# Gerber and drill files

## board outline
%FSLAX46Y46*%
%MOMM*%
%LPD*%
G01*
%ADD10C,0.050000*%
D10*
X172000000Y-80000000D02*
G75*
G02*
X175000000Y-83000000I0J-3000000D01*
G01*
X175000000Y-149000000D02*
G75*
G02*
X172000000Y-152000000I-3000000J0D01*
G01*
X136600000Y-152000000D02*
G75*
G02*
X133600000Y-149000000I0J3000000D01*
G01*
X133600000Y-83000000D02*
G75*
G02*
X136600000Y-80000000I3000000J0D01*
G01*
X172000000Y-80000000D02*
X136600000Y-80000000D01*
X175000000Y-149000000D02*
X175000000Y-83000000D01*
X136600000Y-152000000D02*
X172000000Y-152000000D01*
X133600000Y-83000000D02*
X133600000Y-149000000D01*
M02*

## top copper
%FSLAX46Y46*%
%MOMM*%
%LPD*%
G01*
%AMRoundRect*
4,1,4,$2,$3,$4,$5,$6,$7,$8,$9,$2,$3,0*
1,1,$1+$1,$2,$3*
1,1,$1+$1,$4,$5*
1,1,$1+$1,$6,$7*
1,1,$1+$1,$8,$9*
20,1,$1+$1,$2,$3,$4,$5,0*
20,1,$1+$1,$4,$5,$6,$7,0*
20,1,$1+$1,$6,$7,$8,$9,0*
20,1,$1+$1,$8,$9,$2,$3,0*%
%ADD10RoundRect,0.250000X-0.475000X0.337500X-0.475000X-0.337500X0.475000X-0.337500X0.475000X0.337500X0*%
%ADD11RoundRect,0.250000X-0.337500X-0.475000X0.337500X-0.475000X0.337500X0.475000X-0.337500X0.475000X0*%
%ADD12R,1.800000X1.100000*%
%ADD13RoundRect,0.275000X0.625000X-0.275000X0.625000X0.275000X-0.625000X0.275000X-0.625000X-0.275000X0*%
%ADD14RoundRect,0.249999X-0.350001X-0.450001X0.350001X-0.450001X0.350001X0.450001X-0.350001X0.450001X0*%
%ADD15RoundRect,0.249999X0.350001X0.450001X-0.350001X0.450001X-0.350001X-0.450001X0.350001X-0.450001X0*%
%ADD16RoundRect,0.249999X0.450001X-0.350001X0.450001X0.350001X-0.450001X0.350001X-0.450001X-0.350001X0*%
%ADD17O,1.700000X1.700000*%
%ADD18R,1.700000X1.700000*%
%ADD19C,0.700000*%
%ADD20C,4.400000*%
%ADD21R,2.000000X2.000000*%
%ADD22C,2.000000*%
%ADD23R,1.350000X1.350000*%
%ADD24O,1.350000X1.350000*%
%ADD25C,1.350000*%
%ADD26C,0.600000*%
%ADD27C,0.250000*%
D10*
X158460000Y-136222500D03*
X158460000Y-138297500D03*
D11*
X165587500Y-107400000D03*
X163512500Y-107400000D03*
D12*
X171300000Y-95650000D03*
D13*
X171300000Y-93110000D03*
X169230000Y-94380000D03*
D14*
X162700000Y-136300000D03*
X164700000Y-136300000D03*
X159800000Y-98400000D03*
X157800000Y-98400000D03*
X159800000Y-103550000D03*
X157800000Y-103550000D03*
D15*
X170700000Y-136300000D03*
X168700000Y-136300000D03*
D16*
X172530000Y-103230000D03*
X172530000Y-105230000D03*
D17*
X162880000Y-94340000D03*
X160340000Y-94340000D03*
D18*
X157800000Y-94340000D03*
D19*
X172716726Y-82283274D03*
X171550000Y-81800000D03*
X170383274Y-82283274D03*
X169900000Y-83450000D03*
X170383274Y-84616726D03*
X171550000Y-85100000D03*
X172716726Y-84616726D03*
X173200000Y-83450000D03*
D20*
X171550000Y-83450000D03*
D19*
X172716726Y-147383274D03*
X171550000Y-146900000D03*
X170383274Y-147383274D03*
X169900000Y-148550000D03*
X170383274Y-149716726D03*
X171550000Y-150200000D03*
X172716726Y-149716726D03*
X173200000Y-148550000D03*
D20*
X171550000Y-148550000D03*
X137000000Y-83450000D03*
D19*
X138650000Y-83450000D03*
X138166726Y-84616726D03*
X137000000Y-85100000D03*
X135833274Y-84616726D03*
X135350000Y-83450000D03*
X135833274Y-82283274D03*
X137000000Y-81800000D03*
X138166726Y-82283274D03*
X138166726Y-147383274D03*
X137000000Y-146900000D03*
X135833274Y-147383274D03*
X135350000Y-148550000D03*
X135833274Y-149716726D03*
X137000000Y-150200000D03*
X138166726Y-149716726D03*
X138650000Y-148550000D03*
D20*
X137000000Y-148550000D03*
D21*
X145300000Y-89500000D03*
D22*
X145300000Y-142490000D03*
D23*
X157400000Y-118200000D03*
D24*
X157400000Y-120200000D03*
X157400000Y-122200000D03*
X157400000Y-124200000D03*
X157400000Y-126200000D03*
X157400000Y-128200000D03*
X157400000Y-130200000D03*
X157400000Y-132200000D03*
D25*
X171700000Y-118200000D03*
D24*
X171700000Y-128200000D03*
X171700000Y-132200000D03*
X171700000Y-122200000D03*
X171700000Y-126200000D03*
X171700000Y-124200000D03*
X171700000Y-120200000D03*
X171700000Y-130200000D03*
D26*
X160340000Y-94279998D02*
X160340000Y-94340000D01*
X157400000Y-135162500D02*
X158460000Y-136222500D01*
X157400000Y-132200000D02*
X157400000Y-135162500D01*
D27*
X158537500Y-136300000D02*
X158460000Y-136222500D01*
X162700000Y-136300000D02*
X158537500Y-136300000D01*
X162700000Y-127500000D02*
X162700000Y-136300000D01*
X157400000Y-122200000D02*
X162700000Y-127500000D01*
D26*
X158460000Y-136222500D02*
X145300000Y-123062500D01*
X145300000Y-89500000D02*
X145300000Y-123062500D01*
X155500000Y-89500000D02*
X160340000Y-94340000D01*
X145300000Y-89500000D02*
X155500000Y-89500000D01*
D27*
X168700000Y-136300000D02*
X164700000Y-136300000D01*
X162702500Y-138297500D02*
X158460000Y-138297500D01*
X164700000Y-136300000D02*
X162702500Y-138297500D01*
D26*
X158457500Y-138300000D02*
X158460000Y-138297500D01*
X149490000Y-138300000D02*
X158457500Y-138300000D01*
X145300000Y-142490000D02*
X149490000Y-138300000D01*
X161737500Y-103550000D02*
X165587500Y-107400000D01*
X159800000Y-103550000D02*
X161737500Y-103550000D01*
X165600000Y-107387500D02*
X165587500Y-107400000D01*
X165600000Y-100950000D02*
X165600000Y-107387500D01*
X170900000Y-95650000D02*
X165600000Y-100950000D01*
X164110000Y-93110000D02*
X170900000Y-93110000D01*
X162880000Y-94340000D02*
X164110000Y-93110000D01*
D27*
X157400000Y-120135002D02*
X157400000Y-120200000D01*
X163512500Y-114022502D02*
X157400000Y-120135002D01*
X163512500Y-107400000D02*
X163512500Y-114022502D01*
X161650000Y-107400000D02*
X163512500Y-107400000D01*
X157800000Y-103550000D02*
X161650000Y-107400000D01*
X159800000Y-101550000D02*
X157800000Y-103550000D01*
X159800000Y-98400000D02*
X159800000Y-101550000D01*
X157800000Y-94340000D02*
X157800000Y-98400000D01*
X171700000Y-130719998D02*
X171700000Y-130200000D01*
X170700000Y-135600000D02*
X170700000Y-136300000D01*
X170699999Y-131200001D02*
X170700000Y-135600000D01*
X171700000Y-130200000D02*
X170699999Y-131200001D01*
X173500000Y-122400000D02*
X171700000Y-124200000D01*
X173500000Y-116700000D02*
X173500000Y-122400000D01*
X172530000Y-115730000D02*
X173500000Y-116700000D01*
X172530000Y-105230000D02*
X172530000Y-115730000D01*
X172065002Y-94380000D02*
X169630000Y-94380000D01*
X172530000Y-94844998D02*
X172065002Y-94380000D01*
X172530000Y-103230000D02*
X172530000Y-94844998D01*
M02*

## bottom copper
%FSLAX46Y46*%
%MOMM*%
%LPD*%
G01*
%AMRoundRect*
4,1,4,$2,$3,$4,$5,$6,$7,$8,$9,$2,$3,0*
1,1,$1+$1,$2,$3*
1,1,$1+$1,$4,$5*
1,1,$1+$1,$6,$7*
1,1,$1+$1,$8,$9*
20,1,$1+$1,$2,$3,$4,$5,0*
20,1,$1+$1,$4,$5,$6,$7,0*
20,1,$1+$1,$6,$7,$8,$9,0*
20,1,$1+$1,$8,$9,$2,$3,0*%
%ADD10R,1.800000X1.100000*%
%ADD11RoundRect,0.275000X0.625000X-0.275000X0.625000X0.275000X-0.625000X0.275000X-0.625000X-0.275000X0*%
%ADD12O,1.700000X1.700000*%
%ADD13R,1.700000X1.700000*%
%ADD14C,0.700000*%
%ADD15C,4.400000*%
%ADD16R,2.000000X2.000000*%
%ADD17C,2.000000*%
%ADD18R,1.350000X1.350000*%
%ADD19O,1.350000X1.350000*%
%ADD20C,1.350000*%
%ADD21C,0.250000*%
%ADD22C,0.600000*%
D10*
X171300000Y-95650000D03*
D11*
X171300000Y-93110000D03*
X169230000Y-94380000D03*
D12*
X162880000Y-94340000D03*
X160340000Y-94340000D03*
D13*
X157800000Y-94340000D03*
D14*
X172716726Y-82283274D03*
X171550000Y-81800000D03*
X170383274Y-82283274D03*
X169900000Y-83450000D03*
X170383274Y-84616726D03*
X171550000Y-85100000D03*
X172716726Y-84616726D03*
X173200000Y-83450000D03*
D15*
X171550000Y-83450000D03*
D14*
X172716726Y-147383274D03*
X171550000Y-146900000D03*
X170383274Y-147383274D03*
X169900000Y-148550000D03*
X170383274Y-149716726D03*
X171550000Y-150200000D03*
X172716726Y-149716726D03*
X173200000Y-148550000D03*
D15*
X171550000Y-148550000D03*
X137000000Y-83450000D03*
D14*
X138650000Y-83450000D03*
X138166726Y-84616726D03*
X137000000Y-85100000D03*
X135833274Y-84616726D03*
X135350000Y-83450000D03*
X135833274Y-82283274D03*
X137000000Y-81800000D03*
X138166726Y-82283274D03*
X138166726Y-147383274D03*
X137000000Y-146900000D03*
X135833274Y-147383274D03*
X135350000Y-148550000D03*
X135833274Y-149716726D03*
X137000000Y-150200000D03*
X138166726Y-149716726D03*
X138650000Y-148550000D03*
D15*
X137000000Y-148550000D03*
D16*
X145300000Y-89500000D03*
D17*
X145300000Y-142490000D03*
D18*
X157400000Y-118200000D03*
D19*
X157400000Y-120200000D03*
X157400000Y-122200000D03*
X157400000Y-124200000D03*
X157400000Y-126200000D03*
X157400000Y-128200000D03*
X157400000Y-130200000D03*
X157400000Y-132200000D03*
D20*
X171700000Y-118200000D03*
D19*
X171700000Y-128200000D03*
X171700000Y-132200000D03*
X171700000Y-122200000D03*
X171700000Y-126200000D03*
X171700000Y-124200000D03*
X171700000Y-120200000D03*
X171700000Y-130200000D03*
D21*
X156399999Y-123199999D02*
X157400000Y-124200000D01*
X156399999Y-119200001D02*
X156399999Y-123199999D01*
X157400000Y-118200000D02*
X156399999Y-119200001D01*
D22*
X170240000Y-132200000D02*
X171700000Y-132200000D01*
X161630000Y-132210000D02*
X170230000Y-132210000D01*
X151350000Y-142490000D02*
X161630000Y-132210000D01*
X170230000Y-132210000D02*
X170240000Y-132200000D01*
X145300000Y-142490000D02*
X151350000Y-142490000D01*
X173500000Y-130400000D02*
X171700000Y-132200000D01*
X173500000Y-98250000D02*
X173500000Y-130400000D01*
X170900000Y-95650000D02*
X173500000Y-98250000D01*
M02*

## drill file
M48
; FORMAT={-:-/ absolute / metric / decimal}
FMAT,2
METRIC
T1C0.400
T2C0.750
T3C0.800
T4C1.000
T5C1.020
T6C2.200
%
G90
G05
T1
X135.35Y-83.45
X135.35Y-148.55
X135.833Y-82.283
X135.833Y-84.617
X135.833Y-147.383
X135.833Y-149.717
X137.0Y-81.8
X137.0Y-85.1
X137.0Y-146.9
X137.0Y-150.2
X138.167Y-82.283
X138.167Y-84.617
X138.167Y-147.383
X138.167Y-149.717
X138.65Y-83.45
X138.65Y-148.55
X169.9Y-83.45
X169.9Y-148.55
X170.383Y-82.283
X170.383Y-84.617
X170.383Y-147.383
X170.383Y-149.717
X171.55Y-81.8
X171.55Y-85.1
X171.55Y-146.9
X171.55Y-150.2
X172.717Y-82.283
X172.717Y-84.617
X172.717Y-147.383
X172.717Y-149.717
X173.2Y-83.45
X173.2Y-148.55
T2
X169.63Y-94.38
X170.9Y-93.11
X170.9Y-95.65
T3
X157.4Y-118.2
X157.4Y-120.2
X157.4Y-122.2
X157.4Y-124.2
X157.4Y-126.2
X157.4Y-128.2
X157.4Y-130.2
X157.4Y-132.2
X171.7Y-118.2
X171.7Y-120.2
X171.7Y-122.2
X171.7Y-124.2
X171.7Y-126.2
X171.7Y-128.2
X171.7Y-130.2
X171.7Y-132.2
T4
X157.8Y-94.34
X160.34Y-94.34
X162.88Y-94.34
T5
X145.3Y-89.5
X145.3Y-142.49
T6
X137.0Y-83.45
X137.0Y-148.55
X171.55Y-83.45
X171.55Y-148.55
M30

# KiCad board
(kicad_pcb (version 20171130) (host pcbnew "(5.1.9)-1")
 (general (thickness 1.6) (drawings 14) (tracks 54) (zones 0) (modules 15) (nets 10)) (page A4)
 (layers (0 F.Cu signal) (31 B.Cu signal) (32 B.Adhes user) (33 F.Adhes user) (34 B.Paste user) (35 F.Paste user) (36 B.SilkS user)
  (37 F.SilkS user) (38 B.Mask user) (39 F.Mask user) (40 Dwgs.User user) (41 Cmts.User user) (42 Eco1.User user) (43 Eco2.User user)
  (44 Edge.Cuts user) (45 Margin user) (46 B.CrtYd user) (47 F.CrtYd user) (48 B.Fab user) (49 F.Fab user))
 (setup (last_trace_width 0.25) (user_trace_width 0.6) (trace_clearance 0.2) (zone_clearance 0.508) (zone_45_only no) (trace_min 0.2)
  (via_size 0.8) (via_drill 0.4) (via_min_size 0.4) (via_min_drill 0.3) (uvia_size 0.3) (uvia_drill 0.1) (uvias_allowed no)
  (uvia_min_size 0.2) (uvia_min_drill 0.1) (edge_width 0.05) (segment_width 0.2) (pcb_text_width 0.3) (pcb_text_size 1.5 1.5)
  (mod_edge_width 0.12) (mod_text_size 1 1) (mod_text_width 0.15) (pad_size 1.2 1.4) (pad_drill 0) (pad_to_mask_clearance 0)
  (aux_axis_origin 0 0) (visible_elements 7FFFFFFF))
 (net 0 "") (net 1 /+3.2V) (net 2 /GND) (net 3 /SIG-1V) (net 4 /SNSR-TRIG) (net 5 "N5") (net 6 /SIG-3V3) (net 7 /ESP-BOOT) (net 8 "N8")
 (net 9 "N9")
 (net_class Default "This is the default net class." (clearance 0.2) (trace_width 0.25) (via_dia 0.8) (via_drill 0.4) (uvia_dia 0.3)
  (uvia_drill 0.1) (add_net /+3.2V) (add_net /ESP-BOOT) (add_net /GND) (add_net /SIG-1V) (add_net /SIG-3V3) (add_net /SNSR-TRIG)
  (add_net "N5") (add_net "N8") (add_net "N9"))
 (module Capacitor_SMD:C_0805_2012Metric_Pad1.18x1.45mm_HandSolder (layer F.Cu) (at 158.46 137.26 270)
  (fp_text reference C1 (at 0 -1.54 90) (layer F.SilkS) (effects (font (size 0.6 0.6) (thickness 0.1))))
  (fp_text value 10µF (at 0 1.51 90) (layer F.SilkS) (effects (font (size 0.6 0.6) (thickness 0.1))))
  (pad 1 smd roundrect (at -1.0375 0 270) (size 1.175 1.45) (layers F.Cu F.Paste F.Mask) (roundrect_rratio 0.2127659574468085)
   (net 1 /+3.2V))
  (pad 2 smd roundrect (at 1.0375 0 270) (size 1.175 1.45) (layers F.Cu F.Paste F.Mask) (roundrect_rratio 0.2127659574468085) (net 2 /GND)))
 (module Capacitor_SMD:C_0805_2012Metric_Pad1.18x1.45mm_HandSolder (layer F.Cu) (at 164.55 107.4)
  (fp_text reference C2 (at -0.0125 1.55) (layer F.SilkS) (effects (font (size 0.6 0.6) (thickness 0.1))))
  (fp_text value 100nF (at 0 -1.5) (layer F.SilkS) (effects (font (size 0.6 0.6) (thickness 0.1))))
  (pad 2 smd roundrect (at 1.0375 0) (size 1.175 1.45) (layers F.Cu F.Paste F.Mask) (roundrect_rratio 0.2127659574468085) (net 2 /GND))
  (pad 1 smd roundrect (at -1.0375 0) (size 1.175 1.45) (layers F.Cu F.Paste F.Mask) (roundrect_rratio 0.2127659574468085) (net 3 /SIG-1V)))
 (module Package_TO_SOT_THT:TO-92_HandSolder (layer F.Cu) (at 170.9 95.65 90)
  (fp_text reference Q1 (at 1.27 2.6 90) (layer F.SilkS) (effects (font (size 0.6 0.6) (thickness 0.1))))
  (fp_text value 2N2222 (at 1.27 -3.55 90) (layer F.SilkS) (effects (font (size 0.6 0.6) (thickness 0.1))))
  (pad 1 thru_hole rect (at 0 0 90) (size 1.1 1.8) (drill 0.75 (offset 0 0.4)) (layers *.Cu *.Mask) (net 2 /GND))
  (pad 3 thru_hole roundrect (at 2.54 0 90) (size 1.1 1.8) (drill 0.75 (offset 0 0.4)) (layers *.Cu *.Mask) (roundrect_rratio 0.25)
   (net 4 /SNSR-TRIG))
  (pad 2 thru_hole roundrect (at 1.27 -1.27 90) (size 1.1 1.8) (drill 0.75 (offset 0 -0.4)) (layers *.Cu *.Mask) (roundrect_rratio 0.25)
   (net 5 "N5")))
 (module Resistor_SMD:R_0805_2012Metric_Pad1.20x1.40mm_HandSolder (layer F.Cu) (at 163.7 136.3)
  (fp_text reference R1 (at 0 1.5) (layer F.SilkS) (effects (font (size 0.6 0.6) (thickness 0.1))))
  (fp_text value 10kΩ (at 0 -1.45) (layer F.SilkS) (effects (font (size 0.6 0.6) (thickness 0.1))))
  (pad 1 smd roundrect (at -1 0) (size 1.2 1.4) (layers F.Cu F.Paste F.Mask) (roundrect_rratio 0.2083325) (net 1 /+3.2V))
  (pad 2 smd roundrect (at 1 0) (size 1.2 1.4) (layers F.Cu F.Paste F.Mask) (roundrect_rratio 0.2083325) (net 2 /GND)))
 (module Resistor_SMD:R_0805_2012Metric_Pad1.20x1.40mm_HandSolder (layer F.Cu) (at 158.8 98.4)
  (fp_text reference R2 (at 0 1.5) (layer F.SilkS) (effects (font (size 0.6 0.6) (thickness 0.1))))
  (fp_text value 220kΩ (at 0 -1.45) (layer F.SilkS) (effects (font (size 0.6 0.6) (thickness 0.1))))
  (pad 2 smd roundrect (at 1 0) (size 1.2 1.4) (layers F.Cu F.Paste F.Mask) (roundrect_rratio 0.2083325) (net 3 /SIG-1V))
  (pad 1 smd roundrect (at -1 0) (size 1.2 1.4) (layers F.Cu F.Paste F.Mask) (roundrect_rratio 0.2083325) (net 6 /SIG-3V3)))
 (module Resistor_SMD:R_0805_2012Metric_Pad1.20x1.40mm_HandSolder (layer F.Cu) (at 158.8 103.55)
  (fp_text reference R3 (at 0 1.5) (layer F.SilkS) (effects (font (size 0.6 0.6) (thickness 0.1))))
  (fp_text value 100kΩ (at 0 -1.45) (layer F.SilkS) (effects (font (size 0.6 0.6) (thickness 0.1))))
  (pad 2 smd roundrect (at 1 0) (size 1.2 1.4) (layers F.Cu F.Paste F.Mask) (roundrect_rratio 0.2083325) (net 2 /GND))
  (pad 1 smd roundrect (at -1 0) (size 1.2 1.4) (layers F.Cu F.Paste F.Mask) (roundrect_rratio 0.2083325) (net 3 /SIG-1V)))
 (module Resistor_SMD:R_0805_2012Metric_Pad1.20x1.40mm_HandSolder (layer F.Cu) (at 169.7 136.3 180)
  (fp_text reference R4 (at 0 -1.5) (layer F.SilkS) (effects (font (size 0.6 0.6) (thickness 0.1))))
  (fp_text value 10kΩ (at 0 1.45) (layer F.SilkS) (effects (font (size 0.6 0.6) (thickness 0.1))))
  (pad 1 smd roundrect (at -1 0 180) (size 1.2 1.4) (layers F.Cu F.Paste F.Mask) (roundrect_rratio 0.2083325) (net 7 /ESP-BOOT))
  (pad 2 smd roundrect (at 1 0 180) (size 1.2 1.4) (layers F.Cu F.Paste F.Mask) (roundrect_rratio 0.2083325) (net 2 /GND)))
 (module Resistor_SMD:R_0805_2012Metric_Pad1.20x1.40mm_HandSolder (layer F.Cu) (at 172.53 104.23 90)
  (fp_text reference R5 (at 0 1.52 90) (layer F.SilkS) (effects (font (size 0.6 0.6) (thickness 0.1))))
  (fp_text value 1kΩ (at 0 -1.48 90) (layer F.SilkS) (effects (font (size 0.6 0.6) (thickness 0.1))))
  (pad 2 smd roundrect (at 1 0 90) (size 1.2 1.4) (layers F.Cu F.Paste F.Mask) (roundrect_rratio 0.2083325) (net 5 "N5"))
  (pad 1 smd roundrect (at -1 0 90) (size 1.2 1.4) (layers F.Cu F.Paste F.Mask) (roundrect_rratio 0.2083325) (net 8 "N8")))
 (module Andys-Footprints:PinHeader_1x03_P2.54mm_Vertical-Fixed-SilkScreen (layer F.Cu) (at 157.8 94.34 90)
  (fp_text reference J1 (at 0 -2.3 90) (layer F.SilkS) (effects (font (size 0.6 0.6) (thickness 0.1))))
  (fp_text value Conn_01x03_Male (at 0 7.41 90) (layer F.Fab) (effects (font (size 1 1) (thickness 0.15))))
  (pad 3 thru_hole oval (at 0 5.08 90) (size 1.7 1.7) (drill 1) (layers *.Cu *.Mask) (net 4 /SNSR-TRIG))
  (pad 2 thru_hole oval (at 0 2.54 90) (size 1.7 1.7) (drill 1) (layers *.Cu *.Mask) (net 1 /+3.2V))
  (pad 1 thru_hole rect (at 0 0 90) (size 1.7 1.7) (drill 1) (layers *.Cu *.Mask) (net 6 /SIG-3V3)))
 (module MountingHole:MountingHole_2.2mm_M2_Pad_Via (layer F.Cu) (at 171.55 83.45)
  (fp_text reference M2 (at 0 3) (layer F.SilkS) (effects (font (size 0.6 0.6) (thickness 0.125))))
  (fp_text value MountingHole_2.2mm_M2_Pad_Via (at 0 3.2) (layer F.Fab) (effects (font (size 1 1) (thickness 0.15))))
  (pad 1 thru_hole circle (at 1.166726 -1.166726) (size 0.7 0.7) (drill 0.4) (layers *.Cu *.Mask))
  (pad 1 thru_hole circle (at 0 -1.65) (size 0.7 0.7) (drill 0.4) (layers *.Cu *.Mask))
  (pad 1 thru_hole circle (at -1.166726 -1.166726) (size 0.7 0.7) (drill 0.4) (layers *.Cu *.Mask))
  (pad 1 thru_hole circle (at -1.65 0) (size 0.7 0.7) (drill 0.4) (layers *.Cu *.Mask))
  (pad 1 thru_hole circle (at -1.166726 1.166726) (size 0.7 0.7) (drill 0.4) (layers *.Cu *.Mask))
  (pad 1 thru_hole circle (at 0 1.65) (size 0.7 0.7) (drill 0.4) (layers *.Cu *.Mask))
  (pad 1 thru_hole circle (at 1.166726 1.166726) (size 0.7 0.7) (drill 0.4) (layers *.Cu *.Mask))
  (pad 1 thru_hole circle (at 1.65 0) (size 0.7 0.7) (drill 0.4) (layers *.Cu *.Mask))
  (pad 1 thru_hole circle (at 0 0) (size 4.4 4.4) (drill 2.2) (layers *.Cu *.Mask)))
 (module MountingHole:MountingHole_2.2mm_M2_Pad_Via (layer F.Cu) (at 171.55 148.55)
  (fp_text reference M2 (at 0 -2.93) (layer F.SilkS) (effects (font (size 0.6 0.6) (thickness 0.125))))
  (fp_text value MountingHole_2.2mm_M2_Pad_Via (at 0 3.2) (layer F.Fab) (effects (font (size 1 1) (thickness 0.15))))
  (pad 1 thru_hole circle (at 1.166726 -1.166726) (size 0.7 0.7) (drill 0.4) (layers *.Cu *.Mask))
  (pad 1 thru_hole circle (at 0 -1.65) (size 0.7 0.7) (drill 0.4) (layers *.Cu *.Mask))
  (pad 1 thru_hole circle (at -1.166726 -1.166726) (size 0.7 0.7) (drill 0.4) (layers *.Cu *.Mask))
  (pad 1 thru_hole circle (at -1.65 0) (size 0.7 0.7) (drill 0.4) (layers *.Cu *.Mask))
  (pad 1 thru_hole circle (at -1.166726 1.166726) (size 0.7 0.7) (drill 0.4) (layers *.Cu *.Mask))
  (pad 1 thru_hole circle (at 0 1.65) (size 0.7 0.7) (drill 0.4) (layers *.Cu *.Mask))
  (pad 1 thru_hole circle (at 1.166726 1.166726) (size 0.7 0.7) (drill 0.4) (layers *.Cu *.Mask))
  (pad 1 thru_hole circle (at 1.65 0) (size 0.7 0.7) (drill 0.4) (layers *.Cu *.Mask))
  (pad 1 thru_hole circle (at 0 0) (size 4.4 4.4) (drill 2.2) (layers *.Cu *.Mask)))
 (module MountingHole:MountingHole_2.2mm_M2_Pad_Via (layer F.Cu) (at 137 83.45)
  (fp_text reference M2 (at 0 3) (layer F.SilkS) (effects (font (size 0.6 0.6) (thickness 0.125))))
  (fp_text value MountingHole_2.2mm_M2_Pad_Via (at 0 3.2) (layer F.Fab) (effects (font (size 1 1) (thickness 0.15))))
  (pad 1 thru_hole circle (at 0 0) (size 4.4 4.4) (drill 2.2) (layers *.Cu *.Mask))
  (pad 1 thru_hole circle (at 1.65 0) (size 0.7 0.7) (drill 0.4) (layers *.Cu *.Mask))
  (pad 1 thru_hole circle (at 1.166726 1.166726) (size 0.7 0.7) (drill 0.4) (layers *.Cu *.Mask))
  (pad 1 thru_hole circle (at 0 1.65) (size 0.7 0.7) (drill 0.4) (layers *.Cu *.Mask))
  (pad 1 thru_hole circle (at -1.166726 1.166726) (size 0.7 0.7) (drill 0.4) (layers *.Cu *.Mask))
  (pad 1 thru_hole circle (at -1.65 0) (size 0.7 0.7) (drill 0.4) (layers *.Cu *.Mask))
  (pad 1 thru_hole circle (at -1.166726 -1.166726) (size 0.7 0.7) (drill 0.4) (layers *.Cu *.Mask))
  (pad 1 thru_hole circle (at 0 -1.65) (size 0.7 0.7) (drill 0.4) (layers *.Cu *.Mask))
  (pad 1 thru_hole circle (at 1.166726 -1.166726) (size 0.7 0.7) (drill 0.4) (layers *.Cu *.Mask)))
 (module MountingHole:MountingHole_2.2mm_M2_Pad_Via (layer F.Cu) (at 137 148.55)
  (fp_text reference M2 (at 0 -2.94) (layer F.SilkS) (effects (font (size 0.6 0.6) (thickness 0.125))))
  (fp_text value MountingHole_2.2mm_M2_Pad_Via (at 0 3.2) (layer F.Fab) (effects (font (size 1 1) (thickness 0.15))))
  (pad 1 thru_hole circle (at 1.166726 -1.166726) (size 0.7 0.7) (drill 0.4) (layers *.Cu *.Mask))
  (pad 1 thru_hole circle (at 0 -1.65) (size 0.7 0.7) (drill 0.4) (layers *.Cu *.Mask))
  (pad 1 thru_hole circle (at -1.166726 -1.166726) (size 0.7 0.7) (drill 0.4) (layers *.Cu *.Mask))
  (pad 1 thru_hole circle (at -1.65 0) (size 0.7 0.7) (drill 0.4) (layers *.Cu *.Mask))
  (pad 1 thru_hole circle (at -1.166726 1.166726) (size 0.7 0.7) (drill 0.4) (layers *.Cu *.Mask))
  (pad 1 thru_hole circle (at 0 1.65) (size 0.7 0.7) (drill 0.4) (layers *.Cu *.Mask))
  (pad 1 thru_hole circle (at 1.166726 1.166726) (size 0.7 0.7) (drill 0.4) (layers *.Cu *.Mask))
  (pad 1 thru_hole circle (at 1.65 0) (size 0.7 0.7) (drill 0.4) (layers *.Cu *.Mask))
  (pad 1 thru_hole circle (at 0 0) (size 4.4 4.4) (drill 2.2) (layers *.Cu *.Mask)))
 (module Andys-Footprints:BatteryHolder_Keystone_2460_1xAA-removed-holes (layer F.Cu) (at 145.3 90 270)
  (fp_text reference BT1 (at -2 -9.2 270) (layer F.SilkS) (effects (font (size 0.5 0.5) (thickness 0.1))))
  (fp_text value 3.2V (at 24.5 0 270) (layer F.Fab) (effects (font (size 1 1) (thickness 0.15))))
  (pad 1 thru_hole rect (at -0.5 0 90) (size 2 2) (drill 1.02) (layers *.Cu *.Mask) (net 1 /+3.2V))
  (pad 2 thru_hole circle (at 52.49 0 90) (size 2 2) (drill 1.02) (layers *.Cu *.Mask) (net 2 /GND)))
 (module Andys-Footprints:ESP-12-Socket (layer F.Cu) (at 157.4 118.2)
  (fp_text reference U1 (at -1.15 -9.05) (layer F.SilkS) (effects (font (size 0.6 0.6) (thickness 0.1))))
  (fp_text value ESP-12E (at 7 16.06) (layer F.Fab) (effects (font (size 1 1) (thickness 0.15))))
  (pad 1 thru_hole rect (at 0 0) (size 1.35 1.35) (drill 0.8) (layers *.Cu *.Mask) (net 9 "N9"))
  (pad 2 thru_hole oval (at 0 2) (size 1.35 1.35) (drill 0.8) (layers *.Cu *.Mask) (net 3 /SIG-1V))
  (pad 3 thru_hole oval (at 0 4) (size 1.35 1.35) (drill 0.8) (layers *.Cu *.Mask) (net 1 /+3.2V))
  (pad 4 thru_hole oval (at 0 6) (size 1.35 1.35) (drill 0.8) (layers *.Cu *.Mask) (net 9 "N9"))
  (pad 5 thru_hole oval (at 0 8) (size 1.35 1.35) (drill 0.8) (layers *.Cu *.Mask))
  (pad 6 thru_hole oval (at 0 10) (size 1.35 1.35) (drill 0.8) (layers *.Cu *.Mask))
  (pad 7 thru_hole oval (at 0 12) (size 1.35 1.35) (drill 0.8) (layers *.Cu *.Mask))
  (pad 8 thru_hole oval (at 0 14) (size 1.35 1.35) (drill 0.8) (layers *.Cu *.Mask) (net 1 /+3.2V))
  (pad 22 thru_hole circle (at 14.3 0) (size 1.35 1.35) (drill 0.8) (layers *.Cu *.Mask))
  (pad 17 thru_hole oval (at 14.3 10) (size 1.35 1.35) (drill 0.8) (layers *.Cu *.Mask))
  (pad 15 thru_hole oval (at 14.3 14) (size 1.35 1.35) (drill 0.8) (layers *.Cu *.Mask) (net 2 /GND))
  (pad 20 thru_hole oval (at 14.3 4) (size 1.35 1.35) (drill 0.8) (layers *.Cu *.Mask))
  (pad 18 thru_hole oval (at 14.3 8) (size 1.35 1.35) (drill 0.8) (layers *.Cu *.Mask))
  (pad 19 thru_hole oval (at 14.3 6) (size 1.35 1.35) (drill 0.8) (layers *.Cu *.Mask) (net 8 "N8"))
  (pad 21 thru_hole oval (at 14.3 2) (size 1.35 1.35) (drill 0.8) (layers *.Cu *.Mask))
  (pad 16 thru_hole oval (at 14.3 12) (size 1.35 1.35) (drill 0.8) (layers *.Cu *.Mask) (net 7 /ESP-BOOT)))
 (gr_arc (start 172 83) (end 175 83) (angle -90) (layer Edge.Cuts) (width 0.05))
 (gr_arc (start 172 149) (end 172 152) (angle -90) (layer Edge.Cuts) (width 0.05))
 (gr_arc (start 136.6 149) (end 133.6 149) (angle -90) (layer Edge.Cuts) (width 0.05))
 (gr_arc (start 136.6 83) (end 136.6 80) (angle -90) (layer Edge.Cuts) (width 0.05))
 (gr_line (start 172 80) (end 136.6 80) (layer Edge.Cuts) (width 0.05))
 (gr_line (start 175 149) (end 175 83) (layer Edge.Cuts) (width 0.05))
 (gr_line (start 136.6 152) (end 172 152) (layer Edge.Cuts) (width 0.05))
 (gr_line (start 133.6 83) (end 133.6 149) (layer Edge.Cuts) (width 0.05))
 (segment (start 156.399999 123.199999) (end 157.4 124.2) (width 0.25) (layer B.Cu) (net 9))
 (segment (start 156.399999 119.200001) (end 156.399999 123.199999) (width 0.25) (layer B.Cu) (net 9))
 (segment (start 157.4 118.2) (end 156.399999 119.200001) (width 0.25) (layer B.Cu) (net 9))
 (segment (start 160.34 94.279998) (end 160.34 94.34) (width 0.6) (layer F.Cu) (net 1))
 (segment (start 157.4 135.1625) (end 158.46 136.2225) (width 0.6) (layer F.Cu) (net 1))
 (segment (start 157.4 132.2) (end 157.4 135.1625) (width 0.6) (layer F.Cu) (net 1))
 (segment (start 158.5375 136.3) (end 158.46 136.2225) (width 0.25) (layer F.Cu) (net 1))
 (segment (start 162.7 136.3) (end 158.5375 136.3) (width 0.25) (layer F.Cu) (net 1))
 (segment (start 162.7 127.5) (end 162.7 136.3) (width 0.25) (layer F.Cu) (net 1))
 (segment (start 157.4 122.2) (end 162.7 127.5) (width 0.25) (layer F.Cu) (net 1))
 (segment (start 158.46 136.2225) (end 145.3 123.0625) (width 0.6) (layer F.Cu) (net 1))
 (segment (start 145.3 89.5) (end 145.3 123.0625) (width 0.6) (layer F.Cu) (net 1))
 (segment (start 155.5 89.5) (end 160.34 94.34) (width 0.6) (layer F.Cu) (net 1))
 (segment (start 145.3 89.5) (end 155.5 89.5) (width 0.6) (layer F.Cu) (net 1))
 (segment (start 168.7 136.3) (end 164.7 136.3) (width 0.25) (layer F.Cu) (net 2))
 (segment (start 162.7025 138.2975) (end 158.46 138.2975) (width 0.25) (layer F.Cu) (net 2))
 (segment (start 164.7 136.3) (end 162.7025 138.2975) (width 0.25) (layer F.Cu) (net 2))
 (segment (start 170.24 132.2) (end 171.7 132.2) (width 0.6) (layer B.Cu) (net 2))
 (segment (start 161.63 132.21) (end 170.23 132.21) (width 0.6) (layer B.Cu) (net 2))
 (segment (start 151.35 142.49) (end 161.63 132.21) (width 0.6) (layer B.Cu) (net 2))
 (segment (start 170.23 132.21) (end 170.24 132.2) (width 0.6) (layer B.Cu) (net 2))
 (segment (start 145.3 142.49) (end 151.35 142.49) (width 0.6) (layer B.Cu) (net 2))
 (segment (start 158.4575 138.3) (end 158.46 138.2975) (width 0.6) (layer F.Cu) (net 2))
 (segment (start 149.49 138.3) (end 158.4575 138.3) (width 0.6) (layer F.Cu) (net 2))
 (segment (start 145.3 142.49) (end 149.49 138.3) (width 0.6) (layer F.Cu) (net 2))
 (segment (start 173.5 130.4) (end 171.7 132.2) (width 0.6) (layer B.Cu) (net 2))
 (segment (start 173.5 98.25) (end 173.5 130.4) (width 0.6) (layer B.Cu) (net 2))
 (segment (start 170.9 95.65) (end 173.5 98.25) (width 0.6) (layer B.Cu) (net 2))
 (segment (start 161.7375 103.55) (end 165.5875 107.4) (width 0.6) (layer F.Cu) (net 2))
 (segment (start 159.8 103.55) (end 161.7375 103.55) (width 0.6) (layer F.Cu) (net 2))
 (segment (start 165.6 107.3875) (end 165.5875 107.4) (width 0.6) (layer F.Cu) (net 2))
 (segment (start 165.6 100.95) (end 165.6 107.3875) (width 0.6) (layer F.Cu) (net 2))
 (segment (start 170.9 95.65) (end 165.6 100.95) (width 0.6) (layer F.Cu) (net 2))
 (segment (start 164.11 93.11) (end 170.9 93.11) (width 0.6) (layer F.Cu) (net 4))
 (segment (start 162.88 94.34) (end 164.11 93.11) (width 0.6) (layer F.Cu) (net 4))
 (segment (start 157.4 120.135002) (end 157.4 120.2) (width 0.25) (layer F.Cu) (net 3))
 (segment (start 163.5125 114.022502) (end 157.4 120.135002) (width 0.25) (layer F.Cu) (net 3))
 (segment (start 163.5125 107.4) (end 163.5125 114.022502) (width 0.25) (layer F.Cu) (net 3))
 (segment (start 161.65 107.4) (end 163.5125 107.4) (width 0.25) (layer F.Cu) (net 3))
 (segment (start 157.8 103.55) (end 161.65 107.4) (width 0.25) (layer F.Cu) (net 3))
 (segment (start 159.8 101.55) (end 157.8 103.55) (width 0.25) (layer F.Cu) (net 3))
 (segment (start 159.8 98.4) (end 159.8 101.55) (width 0.25) (layer F.Cu) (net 3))
 (segment (start 157.8 94.34) (end 157.8 98.4) (width 0.25) (layer F.Cu) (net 6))
 (segment (start 171.7 130.719998) (end 171.7 130.2) (width 0.25) (layer F.Cu) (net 7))
 (segment (start 170.7 135.6) (end 170.7 136.3) (width 0.25) (layer F.Cu) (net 7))
 (segment (start 170.699999 131.200001) (end 170.7 135.6) (width 0.25) (layer F.Cu) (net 7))
 (segment (start 171.7 130.2) (end 170.699999 131.200001) (width 0.25) (layer F.Cu) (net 7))
 (segment (start 173.5 122.4) (end 171.7 124.2) (width 0.25) (layer F.Cu) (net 8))
 (segment (start 173.5 116.7) (end 173.5 122.4) (width 0.25) (layer F.Cu) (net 8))
 (segment (start 172.53 115.73) (end 173.5 116.7) (width 0.25) (layer F.Cu) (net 8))
 (segment (start 172.53 105.23) (end 172.53 115.73) (width 0.25) (layer F.Cu) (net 8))
 (segment (start 172.065002 94.38) (end 169.63 94.38) (width 0.25) (layer F.Cu) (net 5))
 (segment (start 172.53 94.844998) (end 172.065002 94.38) (width 0.25) (layer F.Cu) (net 5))
 (segment (start 172.53 103.23) (end 172.53 94.844998) (width 0.25) (layer F.Cu) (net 5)))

